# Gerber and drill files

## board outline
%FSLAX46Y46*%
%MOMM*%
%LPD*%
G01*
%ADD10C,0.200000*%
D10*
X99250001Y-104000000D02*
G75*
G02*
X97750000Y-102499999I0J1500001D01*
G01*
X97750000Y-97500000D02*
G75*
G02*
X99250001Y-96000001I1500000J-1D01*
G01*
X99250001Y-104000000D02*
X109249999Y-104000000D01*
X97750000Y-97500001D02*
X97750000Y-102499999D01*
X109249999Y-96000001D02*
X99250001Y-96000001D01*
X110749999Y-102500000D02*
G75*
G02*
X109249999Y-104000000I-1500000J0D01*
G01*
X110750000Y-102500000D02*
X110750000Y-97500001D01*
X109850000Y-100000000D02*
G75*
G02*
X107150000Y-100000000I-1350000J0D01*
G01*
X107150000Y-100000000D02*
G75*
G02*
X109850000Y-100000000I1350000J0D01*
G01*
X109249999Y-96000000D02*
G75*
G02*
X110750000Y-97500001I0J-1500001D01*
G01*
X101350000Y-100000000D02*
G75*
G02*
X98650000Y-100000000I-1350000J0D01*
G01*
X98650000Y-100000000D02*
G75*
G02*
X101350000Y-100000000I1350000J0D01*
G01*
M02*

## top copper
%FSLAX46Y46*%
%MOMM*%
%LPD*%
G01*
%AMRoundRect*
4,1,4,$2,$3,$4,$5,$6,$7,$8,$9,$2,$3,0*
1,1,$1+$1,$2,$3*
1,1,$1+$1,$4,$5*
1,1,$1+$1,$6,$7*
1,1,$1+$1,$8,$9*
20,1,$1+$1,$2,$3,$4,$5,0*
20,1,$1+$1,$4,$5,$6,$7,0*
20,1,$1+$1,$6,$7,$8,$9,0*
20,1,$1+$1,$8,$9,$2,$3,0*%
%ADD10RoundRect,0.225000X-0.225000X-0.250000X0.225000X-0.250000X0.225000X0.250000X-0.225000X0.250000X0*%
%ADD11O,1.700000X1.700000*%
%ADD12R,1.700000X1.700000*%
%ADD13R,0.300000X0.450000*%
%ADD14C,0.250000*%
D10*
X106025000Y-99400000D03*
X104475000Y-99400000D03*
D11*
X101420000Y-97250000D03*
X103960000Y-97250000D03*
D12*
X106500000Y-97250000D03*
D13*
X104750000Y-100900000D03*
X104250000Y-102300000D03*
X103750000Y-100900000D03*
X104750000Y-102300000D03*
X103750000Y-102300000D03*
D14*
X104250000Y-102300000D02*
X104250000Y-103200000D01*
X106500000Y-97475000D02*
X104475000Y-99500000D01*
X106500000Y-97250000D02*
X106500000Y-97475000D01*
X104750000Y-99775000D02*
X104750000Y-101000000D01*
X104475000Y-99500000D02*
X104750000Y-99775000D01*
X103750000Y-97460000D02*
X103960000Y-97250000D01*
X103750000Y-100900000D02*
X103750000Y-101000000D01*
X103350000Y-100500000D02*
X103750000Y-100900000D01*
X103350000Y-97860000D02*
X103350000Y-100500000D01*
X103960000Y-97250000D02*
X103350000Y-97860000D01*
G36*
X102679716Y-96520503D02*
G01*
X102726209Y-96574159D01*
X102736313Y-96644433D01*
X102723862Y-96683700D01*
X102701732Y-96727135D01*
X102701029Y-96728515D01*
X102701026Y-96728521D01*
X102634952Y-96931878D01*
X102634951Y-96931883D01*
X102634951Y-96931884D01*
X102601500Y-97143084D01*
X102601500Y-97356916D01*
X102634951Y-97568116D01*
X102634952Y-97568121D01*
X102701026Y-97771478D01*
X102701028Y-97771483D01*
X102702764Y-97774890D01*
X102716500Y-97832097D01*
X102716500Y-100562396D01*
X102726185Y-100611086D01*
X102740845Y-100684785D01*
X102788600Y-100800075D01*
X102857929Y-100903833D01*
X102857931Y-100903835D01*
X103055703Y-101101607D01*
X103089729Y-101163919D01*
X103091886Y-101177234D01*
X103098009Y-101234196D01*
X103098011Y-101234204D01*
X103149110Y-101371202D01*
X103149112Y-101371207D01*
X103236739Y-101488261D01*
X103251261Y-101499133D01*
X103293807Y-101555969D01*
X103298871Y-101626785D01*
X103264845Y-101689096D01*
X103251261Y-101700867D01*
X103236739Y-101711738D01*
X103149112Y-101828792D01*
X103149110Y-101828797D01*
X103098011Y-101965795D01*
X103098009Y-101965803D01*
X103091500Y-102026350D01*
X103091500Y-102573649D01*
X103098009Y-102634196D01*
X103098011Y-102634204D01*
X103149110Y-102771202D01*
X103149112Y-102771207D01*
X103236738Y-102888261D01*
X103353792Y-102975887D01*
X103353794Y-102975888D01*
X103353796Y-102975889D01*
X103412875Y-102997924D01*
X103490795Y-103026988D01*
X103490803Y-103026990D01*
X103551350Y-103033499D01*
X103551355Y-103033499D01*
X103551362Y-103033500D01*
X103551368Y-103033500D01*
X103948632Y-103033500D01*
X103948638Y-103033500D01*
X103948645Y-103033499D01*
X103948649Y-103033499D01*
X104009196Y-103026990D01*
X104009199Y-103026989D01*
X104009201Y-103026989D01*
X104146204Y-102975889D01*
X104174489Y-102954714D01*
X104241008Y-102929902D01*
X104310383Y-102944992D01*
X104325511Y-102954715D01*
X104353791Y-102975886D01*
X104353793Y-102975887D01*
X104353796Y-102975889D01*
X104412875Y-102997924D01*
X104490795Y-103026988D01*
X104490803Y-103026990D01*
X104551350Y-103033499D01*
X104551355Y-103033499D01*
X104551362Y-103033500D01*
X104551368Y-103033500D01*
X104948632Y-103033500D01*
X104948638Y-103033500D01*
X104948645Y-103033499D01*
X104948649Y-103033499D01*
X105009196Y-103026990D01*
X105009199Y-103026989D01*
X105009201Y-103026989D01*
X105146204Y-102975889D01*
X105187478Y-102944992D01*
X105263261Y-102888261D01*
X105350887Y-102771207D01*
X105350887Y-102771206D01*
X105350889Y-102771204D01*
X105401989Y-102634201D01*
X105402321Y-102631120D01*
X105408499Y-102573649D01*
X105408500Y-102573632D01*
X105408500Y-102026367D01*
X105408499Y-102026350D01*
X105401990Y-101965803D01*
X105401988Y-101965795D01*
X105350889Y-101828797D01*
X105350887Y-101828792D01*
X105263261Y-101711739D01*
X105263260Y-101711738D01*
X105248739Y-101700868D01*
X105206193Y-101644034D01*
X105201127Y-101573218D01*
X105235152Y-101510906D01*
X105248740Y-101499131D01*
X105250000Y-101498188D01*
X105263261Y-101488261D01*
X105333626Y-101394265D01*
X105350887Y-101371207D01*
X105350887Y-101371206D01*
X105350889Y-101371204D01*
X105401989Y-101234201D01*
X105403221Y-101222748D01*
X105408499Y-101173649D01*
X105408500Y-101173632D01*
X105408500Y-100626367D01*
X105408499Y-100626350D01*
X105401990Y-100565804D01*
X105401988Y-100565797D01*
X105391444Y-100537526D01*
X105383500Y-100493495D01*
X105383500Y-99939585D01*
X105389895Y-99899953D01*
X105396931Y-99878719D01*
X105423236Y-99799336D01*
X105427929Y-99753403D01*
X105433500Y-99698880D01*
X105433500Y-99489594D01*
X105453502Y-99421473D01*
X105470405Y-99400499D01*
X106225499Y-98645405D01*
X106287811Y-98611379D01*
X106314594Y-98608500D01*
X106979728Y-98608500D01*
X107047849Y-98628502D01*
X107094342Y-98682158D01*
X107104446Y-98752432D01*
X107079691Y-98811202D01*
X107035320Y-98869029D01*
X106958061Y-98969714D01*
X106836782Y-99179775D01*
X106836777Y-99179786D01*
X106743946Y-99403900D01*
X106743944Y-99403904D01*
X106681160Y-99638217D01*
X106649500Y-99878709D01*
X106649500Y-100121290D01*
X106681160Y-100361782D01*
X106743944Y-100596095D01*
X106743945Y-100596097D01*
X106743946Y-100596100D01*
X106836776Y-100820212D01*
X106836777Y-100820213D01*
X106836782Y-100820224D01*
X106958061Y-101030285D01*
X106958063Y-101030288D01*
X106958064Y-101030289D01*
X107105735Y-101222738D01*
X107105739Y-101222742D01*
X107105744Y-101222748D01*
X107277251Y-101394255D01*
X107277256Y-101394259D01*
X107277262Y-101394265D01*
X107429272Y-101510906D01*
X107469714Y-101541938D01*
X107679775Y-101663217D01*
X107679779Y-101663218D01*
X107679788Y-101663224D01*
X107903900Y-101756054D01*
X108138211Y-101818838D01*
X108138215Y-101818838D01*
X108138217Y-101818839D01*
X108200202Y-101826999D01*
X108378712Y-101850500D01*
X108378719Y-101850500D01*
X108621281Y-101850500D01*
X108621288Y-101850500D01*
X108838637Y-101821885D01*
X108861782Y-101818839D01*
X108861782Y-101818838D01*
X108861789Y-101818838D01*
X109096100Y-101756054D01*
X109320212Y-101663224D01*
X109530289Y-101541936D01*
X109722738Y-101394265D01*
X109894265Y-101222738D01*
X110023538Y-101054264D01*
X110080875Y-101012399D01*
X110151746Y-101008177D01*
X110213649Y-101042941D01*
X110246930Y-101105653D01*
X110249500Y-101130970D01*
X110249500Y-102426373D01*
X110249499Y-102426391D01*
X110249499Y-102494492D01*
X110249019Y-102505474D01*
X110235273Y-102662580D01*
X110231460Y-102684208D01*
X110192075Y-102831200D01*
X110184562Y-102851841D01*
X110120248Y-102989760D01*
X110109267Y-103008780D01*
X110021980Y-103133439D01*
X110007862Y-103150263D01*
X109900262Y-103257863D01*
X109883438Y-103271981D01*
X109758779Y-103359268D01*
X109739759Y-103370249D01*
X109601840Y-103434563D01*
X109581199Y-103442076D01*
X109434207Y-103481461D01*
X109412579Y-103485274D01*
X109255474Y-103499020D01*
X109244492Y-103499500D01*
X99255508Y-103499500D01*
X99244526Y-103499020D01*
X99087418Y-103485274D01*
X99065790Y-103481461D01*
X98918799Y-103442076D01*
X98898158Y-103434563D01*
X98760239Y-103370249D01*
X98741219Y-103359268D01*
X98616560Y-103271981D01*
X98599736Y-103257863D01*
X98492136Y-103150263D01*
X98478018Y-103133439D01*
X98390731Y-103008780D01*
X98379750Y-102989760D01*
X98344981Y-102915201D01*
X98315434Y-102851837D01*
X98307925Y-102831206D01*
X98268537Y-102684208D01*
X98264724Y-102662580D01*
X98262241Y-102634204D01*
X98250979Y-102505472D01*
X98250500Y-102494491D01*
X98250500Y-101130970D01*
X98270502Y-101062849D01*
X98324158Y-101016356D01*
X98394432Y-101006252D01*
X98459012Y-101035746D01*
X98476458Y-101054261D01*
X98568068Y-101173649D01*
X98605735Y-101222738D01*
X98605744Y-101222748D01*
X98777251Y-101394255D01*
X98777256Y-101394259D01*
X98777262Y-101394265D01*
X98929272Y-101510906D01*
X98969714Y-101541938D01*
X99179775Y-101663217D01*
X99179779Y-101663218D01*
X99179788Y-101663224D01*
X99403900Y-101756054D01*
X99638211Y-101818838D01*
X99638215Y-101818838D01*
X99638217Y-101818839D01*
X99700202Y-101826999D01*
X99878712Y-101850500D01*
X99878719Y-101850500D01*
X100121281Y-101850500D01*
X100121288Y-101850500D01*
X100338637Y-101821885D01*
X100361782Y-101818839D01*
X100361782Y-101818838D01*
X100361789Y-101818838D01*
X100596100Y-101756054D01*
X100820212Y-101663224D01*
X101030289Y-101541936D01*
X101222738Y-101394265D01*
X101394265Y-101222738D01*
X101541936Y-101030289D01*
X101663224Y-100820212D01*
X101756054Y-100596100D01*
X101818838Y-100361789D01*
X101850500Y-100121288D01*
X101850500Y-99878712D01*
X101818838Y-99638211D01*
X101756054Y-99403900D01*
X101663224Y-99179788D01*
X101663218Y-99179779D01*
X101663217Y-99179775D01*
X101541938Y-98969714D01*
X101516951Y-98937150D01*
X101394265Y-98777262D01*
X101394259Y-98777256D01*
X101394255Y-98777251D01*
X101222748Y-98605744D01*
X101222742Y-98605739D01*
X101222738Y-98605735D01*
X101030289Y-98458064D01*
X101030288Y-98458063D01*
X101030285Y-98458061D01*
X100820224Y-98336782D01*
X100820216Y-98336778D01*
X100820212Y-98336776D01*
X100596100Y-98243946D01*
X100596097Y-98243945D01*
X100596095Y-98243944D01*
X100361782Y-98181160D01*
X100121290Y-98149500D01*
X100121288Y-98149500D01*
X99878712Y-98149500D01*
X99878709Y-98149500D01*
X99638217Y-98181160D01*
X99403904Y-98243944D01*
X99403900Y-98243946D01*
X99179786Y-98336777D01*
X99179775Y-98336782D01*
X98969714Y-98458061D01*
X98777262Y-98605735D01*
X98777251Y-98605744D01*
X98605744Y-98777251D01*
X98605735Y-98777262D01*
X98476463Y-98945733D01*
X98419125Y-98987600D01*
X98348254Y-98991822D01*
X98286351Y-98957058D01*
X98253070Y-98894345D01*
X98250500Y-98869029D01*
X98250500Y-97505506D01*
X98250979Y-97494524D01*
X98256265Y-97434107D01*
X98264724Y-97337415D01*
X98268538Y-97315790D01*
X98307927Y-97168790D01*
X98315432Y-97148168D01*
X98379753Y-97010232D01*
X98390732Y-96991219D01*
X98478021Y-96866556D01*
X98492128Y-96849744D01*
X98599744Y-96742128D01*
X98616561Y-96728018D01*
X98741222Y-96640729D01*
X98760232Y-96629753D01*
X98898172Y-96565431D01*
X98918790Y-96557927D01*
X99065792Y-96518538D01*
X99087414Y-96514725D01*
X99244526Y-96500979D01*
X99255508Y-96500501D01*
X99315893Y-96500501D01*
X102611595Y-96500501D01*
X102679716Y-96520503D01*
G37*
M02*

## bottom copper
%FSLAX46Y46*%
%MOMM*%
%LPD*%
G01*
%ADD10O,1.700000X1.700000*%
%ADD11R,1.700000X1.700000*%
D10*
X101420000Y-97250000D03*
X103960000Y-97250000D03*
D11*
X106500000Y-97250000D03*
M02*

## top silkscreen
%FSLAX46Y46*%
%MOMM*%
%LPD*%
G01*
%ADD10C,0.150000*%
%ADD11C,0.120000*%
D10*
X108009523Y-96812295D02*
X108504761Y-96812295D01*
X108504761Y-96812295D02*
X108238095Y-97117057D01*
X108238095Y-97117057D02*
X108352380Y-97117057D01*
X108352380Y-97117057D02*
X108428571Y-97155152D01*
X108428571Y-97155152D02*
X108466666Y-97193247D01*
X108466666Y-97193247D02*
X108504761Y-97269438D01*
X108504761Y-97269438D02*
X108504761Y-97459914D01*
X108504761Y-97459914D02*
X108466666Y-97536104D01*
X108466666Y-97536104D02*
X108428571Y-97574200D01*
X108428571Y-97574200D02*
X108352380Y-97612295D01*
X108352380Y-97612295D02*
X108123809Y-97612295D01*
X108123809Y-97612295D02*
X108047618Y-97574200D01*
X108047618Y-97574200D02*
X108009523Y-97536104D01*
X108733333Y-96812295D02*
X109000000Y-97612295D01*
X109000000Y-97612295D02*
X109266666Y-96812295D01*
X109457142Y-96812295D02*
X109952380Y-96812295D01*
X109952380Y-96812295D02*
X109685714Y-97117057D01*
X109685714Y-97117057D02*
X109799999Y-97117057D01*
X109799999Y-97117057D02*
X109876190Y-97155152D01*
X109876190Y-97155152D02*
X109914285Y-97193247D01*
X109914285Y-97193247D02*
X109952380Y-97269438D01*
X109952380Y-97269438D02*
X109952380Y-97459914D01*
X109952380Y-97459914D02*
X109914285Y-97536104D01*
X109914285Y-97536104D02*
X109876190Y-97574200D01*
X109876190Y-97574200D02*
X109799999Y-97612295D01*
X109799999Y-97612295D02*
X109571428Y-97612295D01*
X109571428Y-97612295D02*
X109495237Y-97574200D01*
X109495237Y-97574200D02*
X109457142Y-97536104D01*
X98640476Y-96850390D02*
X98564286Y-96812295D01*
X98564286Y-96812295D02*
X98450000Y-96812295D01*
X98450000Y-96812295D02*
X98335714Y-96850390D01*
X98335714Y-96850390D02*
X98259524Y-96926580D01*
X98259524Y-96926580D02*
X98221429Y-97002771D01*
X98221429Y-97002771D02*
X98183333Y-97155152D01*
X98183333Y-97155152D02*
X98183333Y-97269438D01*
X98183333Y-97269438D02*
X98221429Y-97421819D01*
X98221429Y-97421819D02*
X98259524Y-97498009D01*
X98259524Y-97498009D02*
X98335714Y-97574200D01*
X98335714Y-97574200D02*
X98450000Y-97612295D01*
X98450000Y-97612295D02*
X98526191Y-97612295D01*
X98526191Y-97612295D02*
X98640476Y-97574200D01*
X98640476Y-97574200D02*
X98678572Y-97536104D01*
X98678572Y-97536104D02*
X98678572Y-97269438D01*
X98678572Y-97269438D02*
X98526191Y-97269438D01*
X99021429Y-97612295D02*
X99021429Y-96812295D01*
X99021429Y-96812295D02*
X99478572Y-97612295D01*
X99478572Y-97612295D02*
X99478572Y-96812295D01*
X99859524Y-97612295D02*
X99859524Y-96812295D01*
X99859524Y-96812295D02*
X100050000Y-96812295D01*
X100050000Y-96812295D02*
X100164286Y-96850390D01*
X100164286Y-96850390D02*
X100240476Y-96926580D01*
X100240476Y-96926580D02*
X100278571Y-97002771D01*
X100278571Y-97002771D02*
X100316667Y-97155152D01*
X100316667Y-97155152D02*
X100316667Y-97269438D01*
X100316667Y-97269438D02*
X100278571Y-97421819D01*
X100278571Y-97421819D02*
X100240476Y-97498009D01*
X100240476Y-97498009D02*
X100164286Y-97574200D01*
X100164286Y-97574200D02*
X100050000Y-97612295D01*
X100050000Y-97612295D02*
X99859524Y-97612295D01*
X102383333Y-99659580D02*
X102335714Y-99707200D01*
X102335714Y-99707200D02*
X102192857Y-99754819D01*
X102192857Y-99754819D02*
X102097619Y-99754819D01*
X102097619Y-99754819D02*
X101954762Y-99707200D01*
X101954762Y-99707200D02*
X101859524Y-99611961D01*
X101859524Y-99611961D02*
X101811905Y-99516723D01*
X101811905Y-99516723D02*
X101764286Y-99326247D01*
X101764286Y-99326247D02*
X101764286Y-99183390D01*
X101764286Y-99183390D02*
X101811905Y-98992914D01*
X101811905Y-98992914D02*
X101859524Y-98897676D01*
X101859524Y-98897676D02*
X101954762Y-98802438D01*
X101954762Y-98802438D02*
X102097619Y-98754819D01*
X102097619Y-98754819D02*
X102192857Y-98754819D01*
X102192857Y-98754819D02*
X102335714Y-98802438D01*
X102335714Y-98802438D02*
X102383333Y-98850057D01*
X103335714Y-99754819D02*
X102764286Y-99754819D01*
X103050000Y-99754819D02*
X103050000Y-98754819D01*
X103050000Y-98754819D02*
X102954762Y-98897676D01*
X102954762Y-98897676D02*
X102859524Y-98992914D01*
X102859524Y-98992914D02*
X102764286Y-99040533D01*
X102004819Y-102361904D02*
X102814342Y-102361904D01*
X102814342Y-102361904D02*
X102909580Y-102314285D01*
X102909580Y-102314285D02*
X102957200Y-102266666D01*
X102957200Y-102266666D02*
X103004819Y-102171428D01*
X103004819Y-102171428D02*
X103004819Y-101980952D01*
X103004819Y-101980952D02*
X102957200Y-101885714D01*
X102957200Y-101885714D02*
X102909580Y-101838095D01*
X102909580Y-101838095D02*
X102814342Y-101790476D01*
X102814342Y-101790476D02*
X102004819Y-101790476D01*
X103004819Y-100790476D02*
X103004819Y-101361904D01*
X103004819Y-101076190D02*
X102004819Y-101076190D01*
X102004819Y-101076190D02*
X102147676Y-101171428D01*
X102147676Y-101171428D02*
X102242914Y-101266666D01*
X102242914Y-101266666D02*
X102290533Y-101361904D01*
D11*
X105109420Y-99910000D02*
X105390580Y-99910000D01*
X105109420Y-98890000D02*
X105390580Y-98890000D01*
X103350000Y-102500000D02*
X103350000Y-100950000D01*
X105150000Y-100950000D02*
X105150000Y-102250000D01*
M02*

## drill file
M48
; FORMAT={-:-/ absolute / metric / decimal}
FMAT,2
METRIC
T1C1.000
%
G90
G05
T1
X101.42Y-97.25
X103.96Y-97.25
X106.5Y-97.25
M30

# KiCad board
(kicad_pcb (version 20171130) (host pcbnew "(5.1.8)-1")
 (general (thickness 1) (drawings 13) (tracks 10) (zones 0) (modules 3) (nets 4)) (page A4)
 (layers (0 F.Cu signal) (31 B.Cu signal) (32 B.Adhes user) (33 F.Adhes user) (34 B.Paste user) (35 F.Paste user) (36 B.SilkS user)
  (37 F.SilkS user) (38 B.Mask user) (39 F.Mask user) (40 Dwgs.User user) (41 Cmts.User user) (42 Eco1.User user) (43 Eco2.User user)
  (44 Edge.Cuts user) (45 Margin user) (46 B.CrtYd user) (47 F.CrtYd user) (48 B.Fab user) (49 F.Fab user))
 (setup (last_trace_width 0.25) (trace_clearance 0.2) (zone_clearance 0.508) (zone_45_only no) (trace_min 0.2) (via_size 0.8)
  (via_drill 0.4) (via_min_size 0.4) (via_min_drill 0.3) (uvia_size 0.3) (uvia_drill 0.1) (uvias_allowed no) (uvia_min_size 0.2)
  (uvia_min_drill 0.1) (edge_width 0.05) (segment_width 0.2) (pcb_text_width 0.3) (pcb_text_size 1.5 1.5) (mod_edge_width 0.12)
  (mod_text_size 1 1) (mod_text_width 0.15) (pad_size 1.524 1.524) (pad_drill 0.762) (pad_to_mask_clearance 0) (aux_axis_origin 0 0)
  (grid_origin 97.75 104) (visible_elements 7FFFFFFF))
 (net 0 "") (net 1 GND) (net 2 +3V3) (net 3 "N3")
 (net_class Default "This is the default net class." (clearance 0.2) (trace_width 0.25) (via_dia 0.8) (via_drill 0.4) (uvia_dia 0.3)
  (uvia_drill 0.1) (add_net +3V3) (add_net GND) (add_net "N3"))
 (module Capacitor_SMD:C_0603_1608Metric (layer F.Cu) (at 105.25 99.4)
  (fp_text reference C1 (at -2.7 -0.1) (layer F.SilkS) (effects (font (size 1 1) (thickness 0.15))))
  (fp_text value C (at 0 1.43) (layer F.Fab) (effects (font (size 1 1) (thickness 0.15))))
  (fp_line (start -0.14058 0.51) (end 0.14058 0.51) (layer F.SilkS) (width 0.12))
  (fp_line (start -0.14058 -0.51) (end 0.14058 -0.51) (layer F.SilkS) (width 0.12))
  (pad 2 smd roundrect (at 0.775 0) (size 0.9 0.95) (layers F.Cu F.Paste F.Mask) (roundrect_rratio 0.25) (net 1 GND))
  (pad 1 smd roundrect (at -0.775 0) (size 0.9 0.95) (layers F.Cu F.Paste F.Mask) (roundrect_rratio 0.25) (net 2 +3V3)))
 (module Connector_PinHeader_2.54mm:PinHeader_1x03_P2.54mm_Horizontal (layer B.Cu) (at 106.5 97.25 90)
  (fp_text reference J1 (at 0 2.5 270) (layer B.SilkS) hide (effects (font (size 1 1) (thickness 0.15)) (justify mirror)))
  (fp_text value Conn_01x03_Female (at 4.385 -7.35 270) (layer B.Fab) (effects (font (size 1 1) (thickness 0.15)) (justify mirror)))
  (pad 3 thru_hole oval (at 0 -5.08 90) (size 1.7 1.7) (drill 1) (layers *.Cu *.Mask) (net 1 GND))
  (pad 2 thru_hole oval (at 0 -2.54 90) (size 1.7 1.7) (drill 1) (layers *.Cu *.Mask) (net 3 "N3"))
  (pad 1 thru_hole rect (at 0 0 90) (size 1.7 1.7) (drill 1) (layers *.Cu *.Mask) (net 2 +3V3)))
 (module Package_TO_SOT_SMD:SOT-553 (layer F.Cu) (at 104.25 101.6 90)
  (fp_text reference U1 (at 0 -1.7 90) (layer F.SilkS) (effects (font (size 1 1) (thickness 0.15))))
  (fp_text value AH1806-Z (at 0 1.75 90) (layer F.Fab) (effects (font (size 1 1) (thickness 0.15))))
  (fp_line (start -0.9 -0.9) (end 0.65 -0.9) (layer F.SilkS) (width 0.12))
  (fp_line (start 0.65 0.9) (end -0.65 0.9) (layer F.SilkS) (width 0.12))
  (pad 4 smd rect (at 0.7 0.5 90) (size 0.45 0.3) (layers F.Cu F.Paste F.Mask) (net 2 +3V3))
  (pad 2 smd rect (at -0.7 0 90) (size 0.45 0.3) (layers F.Cu F.Paste F.Mask) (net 1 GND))
  (pad 5 smd rect (at 0.7 -0.5 90) (size 0.45 0.3) (layers F.Cu F.Paste F.Mask) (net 3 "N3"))
  (pad 3 smd rect (at -0.7 0.5 90) (size 0.45 0.3) (layers F.Cu F.Paste F.Mask))
  (pad 1 smd rect (at -0.7 -0.5 90) (size 0.45 0.3) (layers F.Cu F.Paste F.Mask)))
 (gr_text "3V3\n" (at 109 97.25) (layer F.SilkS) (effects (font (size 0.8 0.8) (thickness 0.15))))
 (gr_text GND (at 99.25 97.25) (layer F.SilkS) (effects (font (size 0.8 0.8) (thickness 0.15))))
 (gr_arc (start 99.250001 102.499999) (end 97.75 102.499999) (angle -90) (layer Edge.Cuts) (width 0.2))
 (gr_arc (start 99.25 97.500001) (end 99.250001 96.000001) (angle -90) (layer Edge.Cuts) (width 0.2))
 (gr_line (start 99.250001 104) (end 109.249999 104) (layer Edge.Cuts) (width 0.2))
 (gr_line (start 97.75 97.500001) (end 97.75 102.499999) (layer Edge.Cuts) (width 0.2))
 (gr_line (start 109.249999 96.000001) (end 99.250001 96.000001) (layer Edge.Cuts) (width 0.2))
 (gr_arc (start 109.249999 102.5) (end 109.249999 104) (angle -90) (layer Edge.Cuts) (width 0.2))
 (gr_line (start 110.75 102.5) (end 110.75 97.500001) (layer Edge.Cuts) (width 0.2))
 (gr_circle (center 108.5 100) (end 109.85 100) (layer Edge.Cuts) (width 0.2))
 (gr_arc (start 109.249999 97.500001) (end 110.75 97.500001) (angle -90) (layer Edge.Cuts) (width 0.2))
 (gr_circle (center 100 100) (end 101.35 100) (layer Edge.Cuts) (width 0.2))
 (segment (start 104.25 102.3) (end 104.25 103.2) (width 0.25) (layer F.Cu) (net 1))
 (segment (start 106.5 97.475) (end 104.475 99.5) (width 0.25) (layer F.Cu) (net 2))
 (segment (start 106.5 97.25) (end 106.5 97.475) (width 0.25) (layer F.Cu) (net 2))
 (segment (start 104.75 99.775) (end 104.75 101) (width 0.25) (layer F.Cu) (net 2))
 (segment (start 104.475 99.5) (end 104.75 99.775) (width 0.25) (layer F.Cu) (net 2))
 (segment (start 103.75 97.46) (end 103.96 97.25) (width 0.25) (layer F.Cu) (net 3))
 (segment (start 103.75 100.9) (end 103.75 101) (width 0.25) (layer F.Cu) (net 3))
 (segment (start 103.35 100.5) (end 103.75 100.9) (width 0.25) (layer F.Cu) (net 3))
 (segment (start 103.35 97.86) (end 103.35 100.5) (width 0.25) (layer F.Cu) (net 3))
 (segment (start 103.96 97.25) (end 103.35 97.86) (width 0.25) (layer F.Cu) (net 3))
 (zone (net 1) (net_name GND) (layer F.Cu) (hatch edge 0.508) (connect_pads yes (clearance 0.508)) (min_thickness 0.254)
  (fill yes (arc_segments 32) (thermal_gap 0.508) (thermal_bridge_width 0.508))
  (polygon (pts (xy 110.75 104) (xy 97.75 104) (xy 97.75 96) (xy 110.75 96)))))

